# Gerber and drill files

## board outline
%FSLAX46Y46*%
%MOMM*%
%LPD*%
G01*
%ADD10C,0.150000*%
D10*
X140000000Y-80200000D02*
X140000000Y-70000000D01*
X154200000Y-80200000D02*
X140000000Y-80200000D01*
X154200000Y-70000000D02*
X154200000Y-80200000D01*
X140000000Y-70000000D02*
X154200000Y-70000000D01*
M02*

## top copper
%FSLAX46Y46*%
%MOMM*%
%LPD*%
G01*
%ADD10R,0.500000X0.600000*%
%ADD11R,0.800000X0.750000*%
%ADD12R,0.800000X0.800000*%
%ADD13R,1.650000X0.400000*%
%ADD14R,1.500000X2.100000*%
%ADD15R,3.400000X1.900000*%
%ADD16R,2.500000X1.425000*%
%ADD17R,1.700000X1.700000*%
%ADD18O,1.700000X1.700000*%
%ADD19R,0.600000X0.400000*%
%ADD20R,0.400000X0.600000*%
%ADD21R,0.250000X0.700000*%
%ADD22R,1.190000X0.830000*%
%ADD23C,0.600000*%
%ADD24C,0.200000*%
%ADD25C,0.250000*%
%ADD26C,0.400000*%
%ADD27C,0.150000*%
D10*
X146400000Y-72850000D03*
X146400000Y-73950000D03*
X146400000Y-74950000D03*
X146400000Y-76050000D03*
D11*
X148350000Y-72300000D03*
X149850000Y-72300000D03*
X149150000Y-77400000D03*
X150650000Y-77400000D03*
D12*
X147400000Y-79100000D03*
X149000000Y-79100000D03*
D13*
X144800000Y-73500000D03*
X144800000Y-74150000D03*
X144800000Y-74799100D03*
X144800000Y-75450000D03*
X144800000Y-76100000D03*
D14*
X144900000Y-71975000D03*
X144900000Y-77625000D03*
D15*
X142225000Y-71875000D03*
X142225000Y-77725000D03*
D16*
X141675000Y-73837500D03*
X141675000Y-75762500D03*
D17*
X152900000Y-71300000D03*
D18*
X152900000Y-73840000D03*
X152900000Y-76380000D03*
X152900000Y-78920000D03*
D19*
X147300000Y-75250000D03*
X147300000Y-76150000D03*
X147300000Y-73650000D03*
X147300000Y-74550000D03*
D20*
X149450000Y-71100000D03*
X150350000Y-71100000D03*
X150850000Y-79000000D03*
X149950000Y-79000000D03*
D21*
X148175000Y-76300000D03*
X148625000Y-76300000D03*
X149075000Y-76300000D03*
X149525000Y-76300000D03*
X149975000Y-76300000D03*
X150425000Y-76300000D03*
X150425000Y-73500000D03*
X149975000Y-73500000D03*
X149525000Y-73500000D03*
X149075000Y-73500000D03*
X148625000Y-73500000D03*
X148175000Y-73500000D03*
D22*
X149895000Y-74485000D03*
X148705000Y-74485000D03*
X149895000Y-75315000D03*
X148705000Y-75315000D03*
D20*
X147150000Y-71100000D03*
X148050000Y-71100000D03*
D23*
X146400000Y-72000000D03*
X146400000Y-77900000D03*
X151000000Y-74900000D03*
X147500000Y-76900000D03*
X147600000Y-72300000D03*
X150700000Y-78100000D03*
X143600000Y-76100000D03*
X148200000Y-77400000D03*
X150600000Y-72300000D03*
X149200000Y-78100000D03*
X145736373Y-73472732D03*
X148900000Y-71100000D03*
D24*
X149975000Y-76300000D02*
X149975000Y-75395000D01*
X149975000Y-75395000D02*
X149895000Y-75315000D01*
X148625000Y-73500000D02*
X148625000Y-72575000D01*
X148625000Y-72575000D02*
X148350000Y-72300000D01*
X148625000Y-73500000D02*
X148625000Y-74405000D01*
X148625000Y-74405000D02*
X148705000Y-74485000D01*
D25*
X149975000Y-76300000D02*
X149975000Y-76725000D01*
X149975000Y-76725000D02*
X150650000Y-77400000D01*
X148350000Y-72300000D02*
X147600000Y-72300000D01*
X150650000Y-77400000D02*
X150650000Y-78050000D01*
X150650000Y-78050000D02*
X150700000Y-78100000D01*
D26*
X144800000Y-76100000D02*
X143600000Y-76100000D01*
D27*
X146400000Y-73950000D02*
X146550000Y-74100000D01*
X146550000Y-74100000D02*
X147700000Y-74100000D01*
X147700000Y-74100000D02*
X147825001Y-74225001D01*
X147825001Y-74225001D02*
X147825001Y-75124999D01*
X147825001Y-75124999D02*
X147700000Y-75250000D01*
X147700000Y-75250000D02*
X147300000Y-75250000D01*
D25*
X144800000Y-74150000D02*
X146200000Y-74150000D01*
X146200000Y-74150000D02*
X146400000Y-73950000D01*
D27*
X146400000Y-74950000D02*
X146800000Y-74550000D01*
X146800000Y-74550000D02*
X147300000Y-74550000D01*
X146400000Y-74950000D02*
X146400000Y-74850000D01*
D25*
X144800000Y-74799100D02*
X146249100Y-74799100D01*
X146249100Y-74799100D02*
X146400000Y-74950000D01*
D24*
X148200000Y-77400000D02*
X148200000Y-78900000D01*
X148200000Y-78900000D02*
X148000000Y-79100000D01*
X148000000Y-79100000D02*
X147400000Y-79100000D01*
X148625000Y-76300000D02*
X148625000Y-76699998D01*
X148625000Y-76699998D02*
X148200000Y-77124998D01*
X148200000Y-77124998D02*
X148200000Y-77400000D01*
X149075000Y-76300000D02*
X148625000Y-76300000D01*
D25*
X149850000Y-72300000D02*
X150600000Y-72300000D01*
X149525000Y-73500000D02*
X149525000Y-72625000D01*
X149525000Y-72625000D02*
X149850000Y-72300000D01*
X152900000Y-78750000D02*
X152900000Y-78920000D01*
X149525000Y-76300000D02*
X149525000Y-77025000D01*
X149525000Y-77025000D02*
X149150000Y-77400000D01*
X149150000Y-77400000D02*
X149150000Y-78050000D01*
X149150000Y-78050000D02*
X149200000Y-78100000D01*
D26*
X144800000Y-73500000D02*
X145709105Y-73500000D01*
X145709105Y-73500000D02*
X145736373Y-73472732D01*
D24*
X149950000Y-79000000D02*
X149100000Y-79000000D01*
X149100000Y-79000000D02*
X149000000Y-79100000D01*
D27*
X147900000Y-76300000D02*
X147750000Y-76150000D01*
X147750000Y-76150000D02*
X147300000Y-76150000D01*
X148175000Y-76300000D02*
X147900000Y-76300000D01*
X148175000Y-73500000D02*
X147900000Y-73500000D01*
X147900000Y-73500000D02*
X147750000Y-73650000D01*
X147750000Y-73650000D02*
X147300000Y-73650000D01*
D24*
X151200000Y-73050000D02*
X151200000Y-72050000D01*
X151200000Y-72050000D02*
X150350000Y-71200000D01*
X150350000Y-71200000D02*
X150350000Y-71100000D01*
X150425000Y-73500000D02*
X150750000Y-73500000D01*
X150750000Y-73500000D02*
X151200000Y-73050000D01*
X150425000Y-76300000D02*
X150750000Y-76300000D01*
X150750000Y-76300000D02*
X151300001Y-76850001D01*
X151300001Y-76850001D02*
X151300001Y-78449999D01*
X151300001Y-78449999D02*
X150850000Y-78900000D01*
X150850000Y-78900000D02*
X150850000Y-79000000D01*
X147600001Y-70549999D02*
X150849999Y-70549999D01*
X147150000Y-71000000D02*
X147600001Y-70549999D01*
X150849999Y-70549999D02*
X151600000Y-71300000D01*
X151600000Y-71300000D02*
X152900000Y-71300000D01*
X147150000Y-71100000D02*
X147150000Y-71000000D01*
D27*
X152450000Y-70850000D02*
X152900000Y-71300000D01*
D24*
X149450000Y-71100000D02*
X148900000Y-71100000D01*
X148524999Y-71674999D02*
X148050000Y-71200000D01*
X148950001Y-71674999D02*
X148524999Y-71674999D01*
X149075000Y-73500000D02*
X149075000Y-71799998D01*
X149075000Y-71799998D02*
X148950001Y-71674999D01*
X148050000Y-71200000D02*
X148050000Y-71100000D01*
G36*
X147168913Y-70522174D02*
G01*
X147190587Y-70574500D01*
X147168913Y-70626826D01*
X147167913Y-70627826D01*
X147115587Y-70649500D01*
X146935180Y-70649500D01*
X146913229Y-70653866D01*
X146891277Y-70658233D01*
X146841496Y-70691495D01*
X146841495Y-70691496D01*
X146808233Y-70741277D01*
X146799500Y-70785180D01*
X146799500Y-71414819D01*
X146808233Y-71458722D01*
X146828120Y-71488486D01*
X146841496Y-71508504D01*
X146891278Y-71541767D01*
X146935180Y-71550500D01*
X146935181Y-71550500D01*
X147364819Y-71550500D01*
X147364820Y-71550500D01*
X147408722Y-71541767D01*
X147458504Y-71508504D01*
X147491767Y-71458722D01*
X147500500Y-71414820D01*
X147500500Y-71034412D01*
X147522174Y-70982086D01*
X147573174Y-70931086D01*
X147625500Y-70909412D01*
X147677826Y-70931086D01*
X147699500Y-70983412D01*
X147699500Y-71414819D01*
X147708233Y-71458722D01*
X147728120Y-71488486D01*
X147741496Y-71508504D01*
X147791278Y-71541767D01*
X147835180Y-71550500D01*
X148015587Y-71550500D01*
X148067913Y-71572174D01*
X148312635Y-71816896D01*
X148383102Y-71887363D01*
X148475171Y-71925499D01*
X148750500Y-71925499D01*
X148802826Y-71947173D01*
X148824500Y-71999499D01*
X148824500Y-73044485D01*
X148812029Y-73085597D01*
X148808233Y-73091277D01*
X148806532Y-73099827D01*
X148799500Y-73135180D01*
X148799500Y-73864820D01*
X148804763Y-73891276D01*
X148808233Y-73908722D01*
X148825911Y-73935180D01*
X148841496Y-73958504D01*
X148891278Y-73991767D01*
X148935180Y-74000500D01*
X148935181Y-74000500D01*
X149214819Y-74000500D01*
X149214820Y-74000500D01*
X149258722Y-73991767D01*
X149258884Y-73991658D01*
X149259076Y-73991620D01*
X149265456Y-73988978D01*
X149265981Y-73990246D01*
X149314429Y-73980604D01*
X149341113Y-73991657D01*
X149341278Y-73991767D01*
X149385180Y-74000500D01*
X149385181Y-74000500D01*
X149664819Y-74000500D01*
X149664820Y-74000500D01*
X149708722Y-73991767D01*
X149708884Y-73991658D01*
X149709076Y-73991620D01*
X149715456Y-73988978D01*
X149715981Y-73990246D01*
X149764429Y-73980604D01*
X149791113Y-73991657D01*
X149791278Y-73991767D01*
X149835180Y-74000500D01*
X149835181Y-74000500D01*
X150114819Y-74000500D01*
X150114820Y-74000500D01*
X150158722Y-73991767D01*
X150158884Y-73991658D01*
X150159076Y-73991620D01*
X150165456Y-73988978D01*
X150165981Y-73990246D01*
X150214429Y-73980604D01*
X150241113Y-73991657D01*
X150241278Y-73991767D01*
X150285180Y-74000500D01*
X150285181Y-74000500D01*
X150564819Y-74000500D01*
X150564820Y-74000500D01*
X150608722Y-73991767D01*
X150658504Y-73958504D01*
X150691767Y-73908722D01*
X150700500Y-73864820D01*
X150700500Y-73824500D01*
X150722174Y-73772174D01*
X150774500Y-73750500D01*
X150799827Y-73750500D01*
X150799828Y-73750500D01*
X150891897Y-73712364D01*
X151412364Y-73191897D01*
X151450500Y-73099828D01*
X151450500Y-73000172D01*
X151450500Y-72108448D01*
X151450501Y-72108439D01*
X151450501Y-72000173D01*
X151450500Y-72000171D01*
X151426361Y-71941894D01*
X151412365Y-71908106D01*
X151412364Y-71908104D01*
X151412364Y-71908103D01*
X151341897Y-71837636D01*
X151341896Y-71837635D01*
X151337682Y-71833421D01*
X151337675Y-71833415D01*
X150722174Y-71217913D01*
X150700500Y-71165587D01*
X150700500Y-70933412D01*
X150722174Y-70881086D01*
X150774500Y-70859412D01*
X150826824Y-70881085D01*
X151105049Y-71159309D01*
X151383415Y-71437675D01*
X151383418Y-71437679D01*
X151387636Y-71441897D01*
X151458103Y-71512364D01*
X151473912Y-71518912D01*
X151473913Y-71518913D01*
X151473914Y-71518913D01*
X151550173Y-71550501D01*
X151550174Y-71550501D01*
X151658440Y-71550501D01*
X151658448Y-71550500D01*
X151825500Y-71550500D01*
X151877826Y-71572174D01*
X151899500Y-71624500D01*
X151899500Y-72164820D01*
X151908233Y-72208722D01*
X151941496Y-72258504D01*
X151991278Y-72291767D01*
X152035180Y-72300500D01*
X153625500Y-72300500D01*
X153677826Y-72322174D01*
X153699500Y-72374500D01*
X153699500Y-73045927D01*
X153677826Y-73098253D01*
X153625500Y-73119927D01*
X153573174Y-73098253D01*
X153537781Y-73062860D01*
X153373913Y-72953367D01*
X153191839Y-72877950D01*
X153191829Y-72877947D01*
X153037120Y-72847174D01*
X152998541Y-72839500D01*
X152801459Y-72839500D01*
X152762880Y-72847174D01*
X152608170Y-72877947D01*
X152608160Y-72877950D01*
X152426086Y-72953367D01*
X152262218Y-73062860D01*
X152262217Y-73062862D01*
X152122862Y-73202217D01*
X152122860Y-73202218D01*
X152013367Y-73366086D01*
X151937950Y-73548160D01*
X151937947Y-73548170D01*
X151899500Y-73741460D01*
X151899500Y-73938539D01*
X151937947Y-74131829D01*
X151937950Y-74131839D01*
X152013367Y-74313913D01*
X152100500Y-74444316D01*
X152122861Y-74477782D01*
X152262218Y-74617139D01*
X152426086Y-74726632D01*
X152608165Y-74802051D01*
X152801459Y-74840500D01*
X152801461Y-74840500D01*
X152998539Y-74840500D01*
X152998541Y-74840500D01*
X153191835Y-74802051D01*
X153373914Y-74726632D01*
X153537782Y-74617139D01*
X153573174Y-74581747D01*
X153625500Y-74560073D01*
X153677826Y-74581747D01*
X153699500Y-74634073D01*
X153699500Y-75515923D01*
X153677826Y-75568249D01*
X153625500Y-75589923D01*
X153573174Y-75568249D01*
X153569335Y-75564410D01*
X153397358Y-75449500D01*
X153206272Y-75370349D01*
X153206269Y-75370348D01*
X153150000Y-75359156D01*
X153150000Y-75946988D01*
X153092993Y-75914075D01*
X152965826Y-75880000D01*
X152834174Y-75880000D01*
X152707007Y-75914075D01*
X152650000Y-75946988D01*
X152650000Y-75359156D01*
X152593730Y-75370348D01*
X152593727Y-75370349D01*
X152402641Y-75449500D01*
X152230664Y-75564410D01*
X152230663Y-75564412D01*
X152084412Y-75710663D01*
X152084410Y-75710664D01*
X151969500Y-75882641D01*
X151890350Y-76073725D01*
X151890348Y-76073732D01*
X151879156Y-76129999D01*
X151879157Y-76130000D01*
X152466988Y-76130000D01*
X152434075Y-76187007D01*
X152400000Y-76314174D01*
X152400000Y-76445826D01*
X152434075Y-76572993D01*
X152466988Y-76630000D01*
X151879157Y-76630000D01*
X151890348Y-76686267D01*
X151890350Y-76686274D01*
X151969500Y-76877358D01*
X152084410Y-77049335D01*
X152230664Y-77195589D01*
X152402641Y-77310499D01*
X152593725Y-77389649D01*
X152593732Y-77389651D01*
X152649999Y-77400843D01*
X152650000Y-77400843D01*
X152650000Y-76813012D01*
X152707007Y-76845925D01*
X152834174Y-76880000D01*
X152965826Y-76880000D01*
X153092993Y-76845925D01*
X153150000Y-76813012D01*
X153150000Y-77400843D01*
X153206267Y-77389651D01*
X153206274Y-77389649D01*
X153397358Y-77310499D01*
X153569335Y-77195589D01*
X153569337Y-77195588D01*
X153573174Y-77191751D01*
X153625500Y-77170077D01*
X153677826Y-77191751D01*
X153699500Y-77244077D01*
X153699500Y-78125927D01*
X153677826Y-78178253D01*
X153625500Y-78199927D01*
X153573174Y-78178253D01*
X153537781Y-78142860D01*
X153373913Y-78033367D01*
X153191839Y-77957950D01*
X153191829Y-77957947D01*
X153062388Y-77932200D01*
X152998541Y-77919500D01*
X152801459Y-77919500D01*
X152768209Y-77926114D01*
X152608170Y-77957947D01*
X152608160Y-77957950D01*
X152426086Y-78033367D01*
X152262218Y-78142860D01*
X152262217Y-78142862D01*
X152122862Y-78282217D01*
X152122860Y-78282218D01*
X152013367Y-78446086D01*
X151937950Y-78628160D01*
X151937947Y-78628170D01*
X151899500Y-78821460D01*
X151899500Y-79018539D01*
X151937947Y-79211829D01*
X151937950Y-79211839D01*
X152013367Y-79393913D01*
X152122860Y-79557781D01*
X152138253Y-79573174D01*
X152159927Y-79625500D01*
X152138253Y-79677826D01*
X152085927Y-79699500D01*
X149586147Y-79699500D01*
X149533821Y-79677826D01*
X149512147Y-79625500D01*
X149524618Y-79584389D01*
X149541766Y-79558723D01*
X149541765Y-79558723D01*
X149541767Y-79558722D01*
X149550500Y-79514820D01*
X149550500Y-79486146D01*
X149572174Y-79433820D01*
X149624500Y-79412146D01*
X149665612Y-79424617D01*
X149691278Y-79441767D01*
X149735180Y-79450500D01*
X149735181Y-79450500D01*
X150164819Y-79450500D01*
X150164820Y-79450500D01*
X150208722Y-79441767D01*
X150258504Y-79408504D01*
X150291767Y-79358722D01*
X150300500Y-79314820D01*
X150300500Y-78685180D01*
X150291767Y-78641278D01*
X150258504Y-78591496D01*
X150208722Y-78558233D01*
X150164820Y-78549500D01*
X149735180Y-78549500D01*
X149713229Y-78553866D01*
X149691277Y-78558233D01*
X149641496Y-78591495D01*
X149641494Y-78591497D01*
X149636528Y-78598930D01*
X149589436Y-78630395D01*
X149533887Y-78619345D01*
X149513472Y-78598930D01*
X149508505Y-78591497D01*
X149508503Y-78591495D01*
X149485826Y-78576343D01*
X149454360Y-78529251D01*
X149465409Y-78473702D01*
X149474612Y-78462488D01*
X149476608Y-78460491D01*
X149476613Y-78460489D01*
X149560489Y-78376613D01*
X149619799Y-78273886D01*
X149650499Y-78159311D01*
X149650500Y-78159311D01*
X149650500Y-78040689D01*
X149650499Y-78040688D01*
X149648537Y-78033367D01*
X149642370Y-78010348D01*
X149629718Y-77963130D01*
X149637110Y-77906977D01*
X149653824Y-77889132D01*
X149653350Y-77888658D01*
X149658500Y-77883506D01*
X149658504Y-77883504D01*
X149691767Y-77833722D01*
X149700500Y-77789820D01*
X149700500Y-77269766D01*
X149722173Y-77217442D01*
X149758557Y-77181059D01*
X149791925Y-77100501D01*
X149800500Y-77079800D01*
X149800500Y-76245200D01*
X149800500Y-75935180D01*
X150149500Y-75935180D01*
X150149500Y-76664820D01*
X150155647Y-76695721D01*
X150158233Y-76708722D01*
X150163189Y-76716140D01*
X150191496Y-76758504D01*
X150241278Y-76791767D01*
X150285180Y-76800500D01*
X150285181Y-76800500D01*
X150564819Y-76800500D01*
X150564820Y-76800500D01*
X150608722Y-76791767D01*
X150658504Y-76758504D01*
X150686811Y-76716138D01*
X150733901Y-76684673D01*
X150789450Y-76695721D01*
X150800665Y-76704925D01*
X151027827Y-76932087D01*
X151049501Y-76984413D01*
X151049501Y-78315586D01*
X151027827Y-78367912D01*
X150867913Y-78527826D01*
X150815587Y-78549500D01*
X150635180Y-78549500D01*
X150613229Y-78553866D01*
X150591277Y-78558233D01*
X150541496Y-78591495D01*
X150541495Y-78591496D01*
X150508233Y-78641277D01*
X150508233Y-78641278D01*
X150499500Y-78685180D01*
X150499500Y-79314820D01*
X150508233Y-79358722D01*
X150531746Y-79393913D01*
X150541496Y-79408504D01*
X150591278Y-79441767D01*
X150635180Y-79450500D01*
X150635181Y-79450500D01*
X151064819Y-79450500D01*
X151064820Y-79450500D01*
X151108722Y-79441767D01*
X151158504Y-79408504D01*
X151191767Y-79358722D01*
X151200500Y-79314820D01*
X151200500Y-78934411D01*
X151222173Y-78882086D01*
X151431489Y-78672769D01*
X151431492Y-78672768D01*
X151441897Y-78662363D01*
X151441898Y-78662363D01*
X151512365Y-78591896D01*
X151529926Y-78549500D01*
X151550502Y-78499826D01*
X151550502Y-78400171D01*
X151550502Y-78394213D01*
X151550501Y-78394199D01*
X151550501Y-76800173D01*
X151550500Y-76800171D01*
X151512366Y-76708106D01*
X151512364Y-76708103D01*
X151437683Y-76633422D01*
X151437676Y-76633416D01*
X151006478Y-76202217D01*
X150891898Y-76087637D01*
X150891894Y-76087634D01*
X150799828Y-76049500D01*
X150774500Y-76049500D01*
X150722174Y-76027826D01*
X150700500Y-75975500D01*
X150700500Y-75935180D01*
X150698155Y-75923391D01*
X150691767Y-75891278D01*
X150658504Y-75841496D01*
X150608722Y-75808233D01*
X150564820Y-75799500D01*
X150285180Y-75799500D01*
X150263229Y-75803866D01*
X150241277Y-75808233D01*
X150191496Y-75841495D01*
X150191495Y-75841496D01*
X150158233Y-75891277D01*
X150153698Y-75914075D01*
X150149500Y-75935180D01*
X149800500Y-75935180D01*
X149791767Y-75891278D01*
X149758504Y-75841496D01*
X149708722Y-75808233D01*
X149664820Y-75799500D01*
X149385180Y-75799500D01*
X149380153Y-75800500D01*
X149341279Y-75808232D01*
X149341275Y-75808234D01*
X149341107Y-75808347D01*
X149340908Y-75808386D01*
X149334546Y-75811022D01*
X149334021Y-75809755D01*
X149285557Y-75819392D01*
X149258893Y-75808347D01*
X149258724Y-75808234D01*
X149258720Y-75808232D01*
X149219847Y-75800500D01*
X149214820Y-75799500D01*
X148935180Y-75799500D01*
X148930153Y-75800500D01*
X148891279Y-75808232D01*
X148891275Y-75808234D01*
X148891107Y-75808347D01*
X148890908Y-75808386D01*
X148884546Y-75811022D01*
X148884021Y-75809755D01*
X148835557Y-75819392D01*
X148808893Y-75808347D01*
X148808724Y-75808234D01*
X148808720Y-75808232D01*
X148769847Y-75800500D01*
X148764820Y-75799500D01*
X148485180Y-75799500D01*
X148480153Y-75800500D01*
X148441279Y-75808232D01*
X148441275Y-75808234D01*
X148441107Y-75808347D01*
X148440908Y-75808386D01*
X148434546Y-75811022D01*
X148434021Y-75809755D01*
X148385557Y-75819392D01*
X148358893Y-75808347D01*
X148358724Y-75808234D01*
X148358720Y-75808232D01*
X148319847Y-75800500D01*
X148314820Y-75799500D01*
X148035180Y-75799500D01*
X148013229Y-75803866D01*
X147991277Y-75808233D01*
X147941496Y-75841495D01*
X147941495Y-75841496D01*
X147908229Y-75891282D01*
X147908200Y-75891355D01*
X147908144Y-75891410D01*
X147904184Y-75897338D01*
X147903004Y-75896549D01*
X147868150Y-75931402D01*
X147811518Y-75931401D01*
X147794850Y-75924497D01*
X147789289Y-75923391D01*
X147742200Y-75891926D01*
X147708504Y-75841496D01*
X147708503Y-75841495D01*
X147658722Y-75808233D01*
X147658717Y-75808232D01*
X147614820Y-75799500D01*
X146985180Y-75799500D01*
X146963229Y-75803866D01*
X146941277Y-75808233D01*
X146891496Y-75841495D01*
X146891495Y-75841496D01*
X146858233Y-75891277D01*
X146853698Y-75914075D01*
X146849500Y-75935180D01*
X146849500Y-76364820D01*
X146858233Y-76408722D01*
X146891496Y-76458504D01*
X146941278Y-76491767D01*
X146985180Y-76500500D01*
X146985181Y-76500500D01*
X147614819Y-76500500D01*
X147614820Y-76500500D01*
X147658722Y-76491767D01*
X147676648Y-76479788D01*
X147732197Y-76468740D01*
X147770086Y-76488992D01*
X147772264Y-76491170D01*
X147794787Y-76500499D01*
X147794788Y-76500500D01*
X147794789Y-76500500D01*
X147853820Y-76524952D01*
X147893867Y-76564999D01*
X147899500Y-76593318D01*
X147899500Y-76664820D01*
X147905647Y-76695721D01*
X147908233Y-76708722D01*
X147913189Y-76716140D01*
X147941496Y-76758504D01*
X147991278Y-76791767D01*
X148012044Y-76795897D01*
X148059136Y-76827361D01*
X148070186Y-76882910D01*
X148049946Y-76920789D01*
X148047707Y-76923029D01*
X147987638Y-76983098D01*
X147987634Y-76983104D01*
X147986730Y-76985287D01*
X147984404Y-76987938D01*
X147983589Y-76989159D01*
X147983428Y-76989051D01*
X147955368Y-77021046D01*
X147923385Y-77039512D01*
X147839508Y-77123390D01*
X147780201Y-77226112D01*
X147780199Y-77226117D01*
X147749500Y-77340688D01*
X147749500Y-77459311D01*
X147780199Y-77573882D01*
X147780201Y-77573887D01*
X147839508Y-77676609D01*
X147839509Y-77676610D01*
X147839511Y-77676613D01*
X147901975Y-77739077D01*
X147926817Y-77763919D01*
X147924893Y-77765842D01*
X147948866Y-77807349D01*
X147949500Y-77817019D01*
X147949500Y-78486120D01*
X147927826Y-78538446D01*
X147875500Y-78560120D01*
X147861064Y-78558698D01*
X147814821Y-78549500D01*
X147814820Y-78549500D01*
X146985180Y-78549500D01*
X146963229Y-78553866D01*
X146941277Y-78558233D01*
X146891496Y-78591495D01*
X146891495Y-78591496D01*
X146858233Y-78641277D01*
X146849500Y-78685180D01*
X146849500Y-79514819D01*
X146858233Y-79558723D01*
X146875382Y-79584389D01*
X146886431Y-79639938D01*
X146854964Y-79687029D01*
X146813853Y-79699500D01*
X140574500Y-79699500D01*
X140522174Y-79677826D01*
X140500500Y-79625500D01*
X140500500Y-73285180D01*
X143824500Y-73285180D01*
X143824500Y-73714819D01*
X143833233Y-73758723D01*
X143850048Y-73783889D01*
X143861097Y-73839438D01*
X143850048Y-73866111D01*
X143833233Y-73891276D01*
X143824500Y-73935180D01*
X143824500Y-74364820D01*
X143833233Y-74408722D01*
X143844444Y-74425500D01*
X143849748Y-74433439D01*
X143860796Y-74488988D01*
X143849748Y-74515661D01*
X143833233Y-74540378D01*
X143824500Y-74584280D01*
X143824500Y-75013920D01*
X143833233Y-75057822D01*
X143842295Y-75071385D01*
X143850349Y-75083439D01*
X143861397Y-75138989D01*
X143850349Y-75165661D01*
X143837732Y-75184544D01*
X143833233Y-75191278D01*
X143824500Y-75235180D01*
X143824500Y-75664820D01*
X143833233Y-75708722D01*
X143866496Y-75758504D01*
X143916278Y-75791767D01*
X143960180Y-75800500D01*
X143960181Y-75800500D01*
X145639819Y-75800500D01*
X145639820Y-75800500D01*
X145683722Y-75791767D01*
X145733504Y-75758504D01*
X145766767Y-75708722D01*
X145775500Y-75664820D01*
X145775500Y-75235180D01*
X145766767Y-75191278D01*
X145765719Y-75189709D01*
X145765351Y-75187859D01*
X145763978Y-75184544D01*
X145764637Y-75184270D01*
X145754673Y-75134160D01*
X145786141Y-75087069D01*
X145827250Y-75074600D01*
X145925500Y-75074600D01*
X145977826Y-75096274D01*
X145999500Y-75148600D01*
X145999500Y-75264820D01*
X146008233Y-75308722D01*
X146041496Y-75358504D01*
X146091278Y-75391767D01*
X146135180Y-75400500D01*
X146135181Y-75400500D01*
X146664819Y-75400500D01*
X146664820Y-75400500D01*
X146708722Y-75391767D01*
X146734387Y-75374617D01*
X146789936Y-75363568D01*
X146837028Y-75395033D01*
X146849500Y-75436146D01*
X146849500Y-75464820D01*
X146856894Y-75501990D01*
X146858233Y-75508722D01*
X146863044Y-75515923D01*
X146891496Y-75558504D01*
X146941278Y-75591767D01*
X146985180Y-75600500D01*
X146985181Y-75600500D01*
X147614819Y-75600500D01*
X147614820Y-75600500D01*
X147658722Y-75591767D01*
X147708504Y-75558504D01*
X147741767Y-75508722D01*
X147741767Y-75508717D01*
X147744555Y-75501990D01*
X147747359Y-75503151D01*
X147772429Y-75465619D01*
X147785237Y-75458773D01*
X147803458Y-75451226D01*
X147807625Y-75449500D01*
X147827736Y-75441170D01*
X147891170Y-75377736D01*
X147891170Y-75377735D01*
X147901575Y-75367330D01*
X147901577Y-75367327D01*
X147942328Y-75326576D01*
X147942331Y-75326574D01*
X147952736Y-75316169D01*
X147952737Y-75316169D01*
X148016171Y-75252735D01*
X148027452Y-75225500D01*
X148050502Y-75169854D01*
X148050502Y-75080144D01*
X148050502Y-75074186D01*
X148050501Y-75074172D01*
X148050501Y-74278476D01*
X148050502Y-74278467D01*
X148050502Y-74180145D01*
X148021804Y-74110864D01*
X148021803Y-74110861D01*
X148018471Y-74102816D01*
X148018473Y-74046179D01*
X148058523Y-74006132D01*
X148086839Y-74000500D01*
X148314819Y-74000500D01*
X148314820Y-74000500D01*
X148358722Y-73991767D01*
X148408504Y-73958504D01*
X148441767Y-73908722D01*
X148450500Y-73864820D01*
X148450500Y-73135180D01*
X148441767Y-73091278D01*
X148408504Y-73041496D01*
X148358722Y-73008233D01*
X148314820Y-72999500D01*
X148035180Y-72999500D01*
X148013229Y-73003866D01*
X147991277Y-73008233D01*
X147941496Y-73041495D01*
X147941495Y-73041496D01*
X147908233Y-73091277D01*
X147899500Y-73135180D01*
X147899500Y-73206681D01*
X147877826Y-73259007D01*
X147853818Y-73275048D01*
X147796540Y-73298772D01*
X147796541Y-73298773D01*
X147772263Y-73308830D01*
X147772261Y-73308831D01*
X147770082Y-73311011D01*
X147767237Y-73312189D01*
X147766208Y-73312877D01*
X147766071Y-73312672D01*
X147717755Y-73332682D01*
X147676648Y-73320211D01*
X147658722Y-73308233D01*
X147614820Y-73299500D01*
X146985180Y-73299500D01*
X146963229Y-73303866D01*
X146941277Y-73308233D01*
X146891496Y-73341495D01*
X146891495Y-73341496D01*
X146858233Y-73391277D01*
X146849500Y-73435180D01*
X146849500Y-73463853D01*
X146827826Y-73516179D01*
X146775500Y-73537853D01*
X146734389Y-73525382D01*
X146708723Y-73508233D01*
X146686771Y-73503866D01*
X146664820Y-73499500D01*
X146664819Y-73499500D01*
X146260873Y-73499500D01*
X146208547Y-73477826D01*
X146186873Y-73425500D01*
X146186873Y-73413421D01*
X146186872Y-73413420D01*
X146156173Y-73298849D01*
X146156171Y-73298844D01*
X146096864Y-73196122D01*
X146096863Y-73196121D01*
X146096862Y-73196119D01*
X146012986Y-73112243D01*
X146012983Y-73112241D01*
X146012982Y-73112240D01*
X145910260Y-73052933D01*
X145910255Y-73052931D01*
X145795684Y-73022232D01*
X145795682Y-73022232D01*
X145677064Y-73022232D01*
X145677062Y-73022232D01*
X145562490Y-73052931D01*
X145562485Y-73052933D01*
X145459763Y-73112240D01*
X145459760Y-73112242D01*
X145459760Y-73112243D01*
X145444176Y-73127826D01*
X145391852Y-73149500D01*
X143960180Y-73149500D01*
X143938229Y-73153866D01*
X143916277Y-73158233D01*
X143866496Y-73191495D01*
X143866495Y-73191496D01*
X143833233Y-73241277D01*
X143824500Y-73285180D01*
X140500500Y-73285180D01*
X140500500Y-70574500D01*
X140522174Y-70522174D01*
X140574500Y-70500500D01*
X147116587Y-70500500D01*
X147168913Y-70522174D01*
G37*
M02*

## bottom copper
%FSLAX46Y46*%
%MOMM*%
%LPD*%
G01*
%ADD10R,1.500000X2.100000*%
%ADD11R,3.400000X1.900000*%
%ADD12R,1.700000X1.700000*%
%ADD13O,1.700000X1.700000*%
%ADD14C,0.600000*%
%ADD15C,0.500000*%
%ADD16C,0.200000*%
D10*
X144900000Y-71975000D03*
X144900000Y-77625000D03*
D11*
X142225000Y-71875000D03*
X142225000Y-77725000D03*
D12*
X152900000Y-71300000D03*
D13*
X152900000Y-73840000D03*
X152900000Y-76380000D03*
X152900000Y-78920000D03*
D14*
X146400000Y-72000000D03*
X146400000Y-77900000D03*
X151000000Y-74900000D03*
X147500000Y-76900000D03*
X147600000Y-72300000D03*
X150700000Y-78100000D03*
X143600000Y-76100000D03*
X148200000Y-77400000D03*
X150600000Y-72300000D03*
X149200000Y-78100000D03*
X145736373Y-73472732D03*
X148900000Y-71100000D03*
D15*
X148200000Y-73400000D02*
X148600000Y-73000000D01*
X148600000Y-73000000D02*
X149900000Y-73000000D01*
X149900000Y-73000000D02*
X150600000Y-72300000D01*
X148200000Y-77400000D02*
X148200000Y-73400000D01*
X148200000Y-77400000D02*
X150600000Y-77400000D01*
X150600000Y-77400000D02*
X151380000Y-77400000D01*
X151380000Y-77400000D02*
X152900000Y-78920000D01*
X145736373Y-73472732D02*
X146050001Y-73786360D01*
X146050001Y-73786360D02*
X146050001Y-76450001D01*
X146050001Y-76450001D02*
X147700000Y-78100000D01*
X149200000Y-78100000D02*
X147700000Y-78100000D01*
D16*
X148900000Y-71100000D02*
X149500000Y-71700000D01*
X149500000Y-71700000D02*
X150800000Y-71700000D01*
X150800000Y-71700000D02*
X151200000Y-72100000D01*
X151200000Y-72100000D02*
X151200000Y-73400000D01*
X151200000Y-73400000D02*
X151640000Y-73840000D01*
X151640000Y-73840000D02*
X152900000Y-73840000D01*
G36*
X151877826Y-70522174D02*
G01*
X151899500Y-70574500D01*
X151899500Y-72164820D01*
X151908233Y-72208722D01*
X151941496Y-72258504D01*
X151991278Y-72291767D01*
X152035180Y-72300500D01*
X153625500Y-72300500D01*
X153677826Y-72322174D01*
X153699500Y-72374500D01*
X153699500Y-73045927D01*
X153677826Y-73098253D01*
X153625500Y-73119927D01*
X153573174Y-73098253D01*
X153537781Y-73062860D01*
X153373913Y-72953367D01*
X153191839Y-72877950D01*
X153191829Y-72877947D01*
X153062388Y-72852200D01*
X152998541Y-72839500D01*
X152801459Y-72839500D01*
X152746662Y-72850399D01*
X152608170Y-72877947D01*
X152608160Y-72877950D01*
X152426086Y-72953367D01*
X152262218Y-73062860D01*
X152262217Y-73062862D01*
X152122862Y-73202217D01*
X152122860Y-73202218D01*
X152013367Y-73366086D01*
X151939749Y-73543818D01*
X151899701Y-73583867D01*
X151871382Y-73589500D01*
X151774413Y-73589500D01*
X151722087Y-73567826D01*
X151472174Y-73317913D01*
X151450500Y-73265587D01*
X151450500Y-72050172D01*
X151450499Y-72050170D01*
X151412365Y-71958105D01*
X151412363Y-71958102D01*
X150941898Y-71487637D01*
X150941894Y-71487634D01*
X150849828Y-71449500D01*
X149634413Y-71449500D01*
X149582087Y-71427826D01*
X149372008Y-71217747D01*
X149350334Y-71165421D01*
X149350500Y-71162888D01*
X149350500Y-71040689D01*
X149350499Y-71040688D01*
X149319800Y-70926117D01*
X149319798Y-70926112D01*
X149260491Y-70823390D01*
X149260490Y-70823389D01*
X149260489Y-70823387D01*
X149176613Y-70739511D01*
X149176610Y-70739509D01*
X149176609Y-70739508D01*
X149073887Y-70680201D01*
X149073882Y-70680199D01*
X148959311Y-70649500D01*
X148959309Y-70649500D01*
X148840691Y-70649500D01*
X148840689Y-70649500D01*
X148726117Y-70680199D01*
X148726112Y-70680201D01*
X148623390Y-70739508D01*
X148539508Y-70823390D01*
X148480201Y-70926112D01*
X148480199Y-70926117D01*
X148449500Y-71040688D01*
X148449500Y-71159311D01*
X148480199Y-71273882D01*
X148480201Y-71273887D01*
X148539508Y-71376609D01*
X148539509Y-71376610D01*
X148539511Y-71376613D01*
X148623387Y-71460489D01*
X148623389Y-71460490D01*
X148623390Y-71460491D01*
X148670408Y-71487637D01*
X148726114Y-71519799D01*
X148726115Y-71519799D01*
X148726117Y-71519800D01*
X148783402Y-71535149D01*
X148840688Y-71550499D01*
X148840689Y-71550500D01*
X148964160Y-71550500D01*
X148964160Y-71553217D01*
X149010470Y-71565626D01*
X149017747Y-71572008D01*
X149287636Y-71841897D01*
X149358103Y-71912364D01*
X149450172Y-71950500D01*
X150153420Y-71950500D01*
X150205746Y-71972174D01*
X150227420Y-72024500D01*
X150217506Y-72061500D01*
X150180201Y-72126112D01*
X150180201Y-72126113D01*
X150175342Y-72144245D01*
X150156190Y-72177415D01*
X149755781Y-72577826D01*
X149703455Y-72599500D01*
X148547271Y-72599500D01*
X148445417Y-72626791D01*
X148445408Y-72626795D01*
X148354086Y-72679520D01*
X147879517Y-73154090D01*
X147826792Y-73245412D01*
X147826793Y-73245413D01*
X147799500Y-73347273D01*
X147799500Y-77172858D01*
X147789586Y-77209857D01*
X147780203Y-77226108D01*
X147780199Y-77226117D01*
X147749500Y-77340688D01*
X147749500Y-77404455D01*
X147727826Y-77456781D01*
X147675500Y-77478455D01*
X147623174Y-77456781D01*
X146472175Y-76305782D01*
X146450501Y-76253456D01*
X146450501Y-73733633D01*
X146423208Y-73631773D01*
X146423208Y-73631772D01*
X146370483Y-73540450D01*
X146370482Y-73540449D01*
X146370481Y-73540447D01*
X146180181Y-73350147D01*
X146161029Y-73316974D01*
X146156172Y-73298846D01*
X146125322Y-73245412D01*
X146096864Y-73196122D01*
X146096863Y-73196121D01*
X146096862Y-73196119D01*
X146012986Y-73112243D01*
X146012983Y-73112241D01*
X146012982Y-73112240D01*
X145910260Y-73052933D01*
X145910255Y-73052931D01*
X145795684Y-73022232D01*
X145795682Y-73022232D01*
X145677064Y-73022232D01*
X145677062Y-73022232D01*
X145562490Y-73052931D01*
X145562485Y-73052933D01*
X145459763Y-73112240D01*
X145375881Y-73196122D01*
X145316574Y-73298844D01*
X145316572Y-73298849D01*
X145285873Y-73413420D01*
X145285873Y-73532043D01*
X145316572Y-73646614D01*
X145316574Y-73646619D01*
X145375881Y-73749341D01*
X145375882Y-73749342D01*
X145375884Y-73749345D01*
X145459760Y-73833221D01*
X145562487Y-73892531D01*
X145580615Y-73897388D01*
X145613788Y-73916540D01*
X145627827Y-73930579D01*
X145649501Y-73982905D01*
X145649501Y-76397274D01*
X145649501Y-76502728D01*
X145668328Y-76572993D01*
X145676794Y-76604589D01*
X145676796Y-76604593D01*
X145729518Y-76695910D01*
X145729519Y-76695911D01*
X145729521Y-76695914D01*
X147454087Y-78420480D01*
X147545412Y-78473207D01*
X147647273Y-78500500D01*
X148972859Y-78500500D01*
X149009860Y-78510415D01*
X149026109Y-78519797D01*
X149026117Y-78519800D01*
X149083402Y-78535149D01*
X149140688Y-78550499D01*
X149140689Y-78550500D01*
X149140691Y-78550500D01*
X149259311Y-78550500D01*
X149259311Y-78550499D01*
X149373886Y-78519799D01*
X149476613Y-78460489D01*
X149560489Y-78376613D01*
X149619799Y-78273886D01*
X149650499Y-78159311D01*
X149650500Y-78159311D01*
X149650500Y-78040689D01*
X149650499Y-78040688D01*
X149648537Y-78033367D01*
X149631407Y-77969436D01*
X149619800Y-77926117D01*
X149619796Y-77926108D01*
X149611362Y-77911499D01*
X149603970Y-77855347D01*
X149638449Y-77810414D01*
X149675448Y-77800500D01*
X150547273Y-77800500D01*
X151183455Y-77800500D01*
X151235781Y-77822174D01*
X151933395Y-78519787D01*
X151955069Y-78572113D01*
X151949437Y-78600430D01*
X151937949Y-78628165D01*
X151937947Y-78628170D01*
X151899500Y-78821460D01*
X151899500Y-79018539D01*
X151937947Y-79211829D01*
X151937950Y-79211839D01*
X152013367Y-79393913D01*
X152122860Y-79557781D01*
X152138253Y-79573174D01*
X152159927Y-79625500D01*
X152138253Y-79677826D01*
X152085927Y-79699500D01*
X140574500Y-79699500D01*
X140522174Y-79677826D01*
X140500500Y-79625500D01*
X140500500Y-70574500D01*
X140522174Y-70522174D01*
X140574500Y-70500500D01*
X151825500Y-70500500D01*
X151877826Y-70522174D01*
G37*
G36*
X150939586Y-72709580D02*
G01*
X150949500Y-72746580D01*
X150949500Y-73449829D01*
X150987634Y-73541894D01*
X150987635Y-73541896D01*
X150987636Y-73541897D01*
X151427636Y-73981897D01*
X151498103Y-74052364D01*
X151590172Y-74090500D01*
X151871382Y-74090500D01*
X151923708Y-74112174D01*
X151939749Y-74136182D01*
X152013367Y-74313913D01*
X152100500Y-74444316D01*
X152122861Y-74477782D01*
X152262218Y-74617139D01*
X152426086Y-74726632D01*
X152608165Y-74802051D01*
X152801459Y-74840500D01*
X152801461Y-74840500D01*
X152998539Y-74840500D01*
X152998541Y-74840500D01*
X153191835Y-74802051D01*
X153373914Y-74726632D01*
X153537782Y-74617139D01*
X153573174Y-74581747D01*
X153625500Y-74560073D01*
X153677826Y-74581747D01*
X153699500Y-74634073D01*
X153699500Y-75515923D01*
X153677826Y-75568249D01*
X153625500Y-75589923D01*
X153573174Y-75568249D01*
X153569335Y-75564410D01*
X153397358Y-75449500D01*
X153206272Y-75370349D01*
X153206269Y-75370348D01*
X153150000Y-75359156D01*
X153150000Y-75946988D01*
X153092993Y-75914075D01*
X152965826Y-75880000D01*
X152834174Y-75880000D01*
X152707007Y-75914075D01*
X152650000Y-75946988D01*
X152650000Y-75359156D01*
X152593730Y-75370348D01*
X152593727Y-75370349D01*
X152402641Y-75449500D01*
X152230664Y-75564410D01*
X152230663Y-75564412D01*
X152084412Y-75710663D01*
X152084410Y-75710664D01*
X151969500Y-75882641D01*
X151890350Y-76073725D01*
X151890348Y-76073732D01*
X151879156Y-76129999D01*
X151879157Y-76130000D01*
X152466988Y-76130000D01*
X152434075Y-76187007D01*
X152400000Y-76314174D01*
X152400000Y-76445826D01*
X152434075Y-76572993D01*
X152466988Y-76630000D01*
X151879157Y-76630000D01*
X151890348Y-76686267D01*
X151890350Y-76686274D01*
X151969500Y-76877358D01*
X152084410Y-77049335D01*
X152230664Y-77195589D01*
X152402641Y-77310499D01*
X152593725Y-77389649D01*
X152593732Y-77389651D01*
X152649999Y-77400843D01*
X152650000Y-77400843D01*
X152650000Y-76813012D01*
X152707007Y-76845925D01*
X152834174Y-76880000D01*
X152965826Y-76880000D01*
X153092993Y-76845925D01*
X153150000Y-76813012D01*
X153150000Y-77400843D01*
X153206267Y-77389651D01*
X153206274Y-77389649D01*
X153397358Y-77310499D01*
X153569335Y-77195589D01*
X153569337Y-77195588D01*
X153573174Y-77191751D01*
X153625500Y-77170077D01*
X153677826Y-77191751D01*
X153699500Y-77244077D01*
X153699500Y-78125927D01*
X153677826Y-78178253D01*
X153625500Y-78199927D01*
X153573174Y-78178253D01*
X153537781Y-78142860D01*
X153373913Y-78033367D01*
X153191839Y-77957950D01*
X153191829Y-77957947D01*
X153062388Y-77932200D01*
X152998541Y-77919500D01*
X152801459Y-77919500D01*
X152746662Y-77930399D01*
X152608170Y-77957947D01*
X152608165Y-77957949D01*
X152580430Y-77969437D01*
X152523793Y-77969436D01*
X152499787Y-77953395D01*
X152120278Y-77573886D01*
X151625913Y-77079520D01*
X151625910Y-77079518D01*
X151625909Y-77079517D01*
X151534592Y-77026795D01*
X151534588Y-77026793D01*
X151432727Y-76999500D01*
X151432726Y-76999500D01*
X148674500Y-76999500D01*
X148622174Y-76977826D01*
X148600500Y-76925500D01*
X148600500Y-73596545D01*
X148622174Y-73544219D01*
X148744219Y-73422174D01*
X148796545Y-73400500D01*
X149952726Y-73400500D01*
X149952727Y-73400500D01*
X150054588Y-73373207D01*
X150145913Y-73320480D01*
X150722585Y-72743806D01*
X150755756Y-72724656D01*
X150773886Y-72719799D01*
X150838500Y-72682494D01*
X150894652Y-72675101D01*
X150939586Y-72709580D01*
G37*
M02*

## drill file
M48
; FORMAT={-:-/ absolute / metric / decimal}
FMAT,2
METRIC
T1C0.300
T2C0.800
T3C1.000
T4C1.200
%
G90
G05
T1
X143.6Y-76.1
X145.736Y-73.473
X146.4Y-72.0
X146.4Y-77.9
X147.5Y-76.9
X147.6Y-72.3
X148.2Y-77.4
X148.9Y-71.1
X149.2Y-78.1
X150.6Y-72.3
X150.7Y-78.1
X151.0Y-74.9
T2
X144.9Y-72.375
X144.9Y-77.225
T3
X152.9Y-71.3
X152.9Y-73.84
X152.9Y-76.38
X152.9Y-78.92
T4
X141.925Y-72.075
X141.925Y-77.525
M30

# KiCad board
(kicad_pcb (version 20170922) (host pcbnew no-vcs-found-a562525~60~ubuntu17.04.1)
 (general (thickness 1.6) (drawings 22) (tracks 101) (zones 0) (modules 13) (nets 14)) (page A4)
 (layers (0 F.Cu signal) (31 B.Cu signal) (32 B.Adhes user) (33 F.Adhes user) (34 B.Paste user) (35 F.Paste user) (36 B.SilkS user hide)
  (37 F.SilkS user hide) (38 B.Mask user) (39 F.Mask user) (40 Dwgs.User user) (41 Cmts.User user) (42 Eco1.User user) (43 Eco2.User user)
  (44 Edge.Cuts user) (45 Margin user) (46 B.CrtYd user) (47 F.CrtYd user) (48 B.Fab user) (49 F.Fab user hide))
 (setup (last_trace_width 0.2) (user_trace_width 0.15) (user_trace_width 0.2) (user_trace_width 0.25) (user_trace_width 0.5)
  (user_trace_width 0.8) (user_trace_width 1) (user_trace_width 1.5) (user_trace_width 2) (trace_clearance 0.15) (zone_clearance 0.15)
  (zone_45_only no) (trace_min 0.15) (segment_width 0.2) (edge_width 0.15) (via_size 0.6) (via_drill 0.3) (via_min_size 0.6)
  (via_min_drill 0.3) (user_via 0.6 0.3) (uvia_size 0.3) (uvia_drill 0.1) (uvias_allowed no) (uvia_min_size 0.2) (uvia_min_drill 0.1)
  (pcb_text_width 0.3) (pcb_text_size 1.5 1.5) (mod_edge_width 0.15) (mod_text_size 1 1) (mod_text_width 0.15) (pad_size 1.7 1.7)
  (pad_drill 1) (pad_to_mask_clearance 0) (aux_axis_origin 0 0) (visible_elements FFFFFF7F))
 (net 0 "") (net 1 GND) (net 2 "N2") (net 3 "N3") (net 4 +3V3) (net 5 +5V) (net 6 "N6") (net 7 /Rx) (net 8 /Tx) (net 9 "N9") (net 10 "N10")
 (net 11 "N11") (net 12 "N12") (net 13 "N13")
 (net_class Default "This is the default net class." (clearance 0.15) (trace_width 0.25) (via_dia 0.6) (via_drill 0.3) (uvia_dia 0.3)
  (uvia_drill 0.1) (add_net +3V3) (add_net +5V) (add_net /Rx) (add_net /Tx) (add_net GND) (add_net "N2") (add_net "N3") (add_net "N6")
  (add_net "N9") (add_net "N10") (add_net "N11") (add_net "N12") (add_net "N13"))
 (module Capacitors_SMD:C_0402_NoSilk (layer F.Cu) (at 146.4 73.4 90)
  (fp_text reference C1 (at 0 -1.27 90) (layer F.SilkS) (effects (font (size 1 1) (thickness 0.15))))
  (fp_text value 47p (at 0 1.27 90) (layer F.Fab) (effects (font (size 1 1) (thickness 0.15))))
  (pad 2 smd rect (at 0.55 0 90) (size 0.6 0.5) (layers F.Cu F.Paste F.Mask) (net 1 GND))
  (pad 1 smd rect (at -0.55 0 90) (size 0.6 0.5) (layers F.Cu F.Paste F.Mask) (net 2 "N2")))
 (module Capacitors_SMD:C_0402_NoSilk (layer F.Cu) (at 146.4 75.5 270)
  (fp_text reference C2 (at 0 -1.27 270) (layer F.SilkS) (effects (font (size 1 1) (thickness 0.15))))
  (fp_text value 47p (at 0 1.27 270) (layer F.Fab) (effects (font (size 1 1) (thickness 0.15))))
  (pad 1 smd rect (at -0.55 0 270) (size 0.6 0.5) (layers F.Cu F.Paste F.Mask) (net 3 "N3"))
  (pad 2 smd rect (at 0.55 0 270) (size 0.6 0.5) (layers F.Cu F.Paste F.Mask) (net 1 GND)))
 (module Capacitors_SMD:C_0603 (layer F.Cu) (at 149.1 72.3 180)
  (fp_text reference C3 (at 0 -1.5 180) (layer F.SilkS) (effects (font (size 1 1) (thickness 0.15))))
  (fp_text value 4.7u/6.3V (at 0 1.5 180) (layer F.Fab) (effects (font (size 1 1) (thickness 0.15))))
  (pad 2 smd rect (at 0.75 0 180) (size 0.8 0.75) (layers F.Cu F.Paste F.Mask) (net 1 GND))
  (pad 1 smd rect (at -0.75 0 180) (size 0.8 0.75) (layers F.Cu F.Paste F.Mask) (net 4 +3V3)))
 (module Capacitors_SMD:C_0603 (layer F.Cu) (at 149.9 77.4)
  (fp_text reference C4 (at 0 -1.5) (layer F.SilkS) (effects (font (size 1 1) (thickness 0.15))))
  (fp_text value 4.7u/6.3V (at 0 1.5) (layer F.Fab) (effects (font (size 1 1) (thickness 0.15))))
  (pad 1 smd rect (at -0.75 0) (size 0.8 0.75) (layers F.Cu F.Paste F.Mask) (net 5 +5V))
  (pad 2 smd rect (at 0.75 0) (size 0.8 0.75) (layers F.Cu F.Paste F.Mask) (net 1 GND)))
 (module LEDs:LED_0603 (layer F.Cu) (at 148.2 79.1 180)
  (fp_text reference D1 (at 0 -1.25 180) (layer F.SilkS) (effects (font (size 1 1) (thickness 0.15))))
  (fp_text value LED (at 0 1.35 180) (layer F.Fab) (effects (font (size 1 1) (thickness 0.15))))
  (pad 2 smd rect (at 0.8 0) (size 0.8 0.8) (layers F.Cu F.Paste F.Mask) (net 4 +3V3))
  (pad 1 smd rect (at -0.8 0) (size 0.8 0.8) (layers F.Cu F.Paste F.Mask) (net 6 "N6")))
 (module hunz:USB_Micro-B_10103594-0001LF (layer F.Cu) (at 142.8 74.8 180)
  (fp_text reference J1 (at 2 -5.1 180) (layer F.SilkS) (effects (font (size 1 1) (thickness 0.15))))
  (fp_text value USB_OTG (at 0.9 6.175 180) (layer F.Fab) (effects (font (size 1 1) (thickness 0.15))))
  (pad 1 smd rect (at -2 1.3) (size 1.65 0.4) (layers F.Cu F.Paste F.Mask) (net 5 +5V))
  (pad 2 smd rect (at -2 0.65) (size 1.65 0.4) (layers F.Cu F.Paste F.Mask) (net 2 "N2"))
  (pad 3 smd rect (at -2 0.0009) (size 1.65 0.4) (layers F.Cu F.Paste F.Mask) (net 3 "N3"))
  (pad 4 smd rect (at -2 -0.65) (size 1.65 0.4) (layers F.Cu F.Paste F.Mask))
  (pad 5 smd rect (at -2 -1.3) (size 1.65 0.4) (layers F.Cu F.Paste F.Mask) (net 1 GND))
  (pad 6 thru_hole rect (at -2.1 2.425) (size 1.5 2.1) (drill 0.8 (offset 0 -0.4)) (layers *.Cu *.Mask F.Paste) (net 1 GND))
  (pad 6 thru_hole rect (at -2.1 -2.425) (size 1.5 2.1) (drill 0.8 (offset 0 0.4)) (layers *.Cu *.Mask F.Paste) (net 1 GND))
  (pad 6 thru_hole rect (at 0.875 2.725) (size 3.4 1.9) (drill 1.2 (offset 0.3 -0.2)) (layers *.Cu *.Mask F.Paste) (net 1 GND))
  (pad 6 thru_hole rect (at 0.875 -2.725) (size 3.4 1.9) (drill 1.2 (offset 0.3 0.2)) (layers *.Cu *.Mask F.Paste) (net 1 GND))
  (pad 6 smd rect (at 1.125 0.9625) (size 2.5 1.425) (layers F.Cu F.Paste F.Mask) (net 1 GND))
  (pad 6 smd rect (at 1.125 -0.9625) (size 2.5 1.425) (layers F.Cu F.Paste F.Mask) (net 1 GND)))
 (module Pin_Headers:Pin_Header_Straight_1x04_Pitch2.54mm (layer F.Cu) (at 152.9 71.3)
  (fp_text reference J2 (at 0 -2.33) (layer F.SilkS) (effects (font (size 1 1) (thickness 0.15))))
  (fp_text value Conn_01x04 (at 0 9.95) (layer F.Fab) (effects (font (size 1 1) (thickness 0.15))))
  (pad 1 thru_hole rect (at 0 0) (size 1.7 1.7) (drill 1) (layers *.Cu *.Mask) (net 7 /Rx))
  (pad 2 thru_hole oval (at 0 2.54) (size 1.7 1.7) (drill 1) (layers *.Cu *.Mask) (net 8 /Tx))
  (pad 3 thru_hole oval (at 0 5.08) (size 1.7 1.7) (drill 1) (layers *.Cu *.Mask) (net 1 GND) (zone_connect 1) (thermal_width 0.5)
   (thermal_gap 0.2))
  (pad 4 thru_hole oval (at 0 7.62) (size 1.7 1.7) (drill 1) (layers *.Cu *.Mask) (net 4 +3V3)))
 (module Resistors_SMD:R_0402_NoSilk (layer F.Cu) (at 147.3 75.7 90)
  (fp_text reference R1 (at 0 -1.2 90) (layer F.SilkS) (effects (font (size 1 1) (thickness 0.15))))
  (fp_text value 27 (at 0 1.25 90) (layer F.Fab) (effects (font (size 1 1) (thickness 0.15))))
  (pad 2 smd rect (at 0.45 0 90) (size 0.4 0.6) (layers F.Cu F.Paste F.Mask) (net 2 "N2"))
  (pad 1 smd rect (at -0.45 0 90) (size 0.4 0.6) (layers F.Cu F.Paste F.Mask) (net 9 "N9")))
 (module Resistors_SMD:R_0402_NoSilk (layer F.Cu) (at 147.3 74.1 270)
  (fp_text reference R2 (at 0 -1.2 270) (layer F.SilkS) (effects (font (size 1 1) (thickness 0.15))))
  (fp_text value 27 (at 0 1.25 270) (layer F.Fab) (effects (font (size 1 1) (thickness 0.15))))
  (pad 1 smd rect (at -0.45 0 270) (size 0.4 0.6) (layers F.Cu F.Paste F.Mask) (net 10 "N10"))
  (pad 2 smd rect (at 0.45 0 270) (size 0.4 0.6) (layers F.Cu F.Paste F.Mask) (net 3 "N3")))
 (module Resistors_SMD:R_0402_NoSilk (layer F.Cu) (at 149.9 71.1)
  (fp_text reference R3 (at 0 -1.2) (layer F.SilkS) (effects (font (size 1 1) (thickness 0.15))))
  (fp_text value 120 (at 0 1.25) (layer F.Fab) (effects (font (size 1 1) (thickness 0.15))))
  (pad 1 smd rect (at -0.45 0) (size 0.4 0.6) (layers F.Cu F.Paste F.Mask) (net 8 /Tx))
  (pad 2 smd rect (at 0.45 0) (size 0.4 0.6) (layers F.Cu F.Paste F.Mask) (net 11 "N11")))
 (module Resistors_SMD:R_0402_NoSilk (layer F.Cu) (at 150.4 79)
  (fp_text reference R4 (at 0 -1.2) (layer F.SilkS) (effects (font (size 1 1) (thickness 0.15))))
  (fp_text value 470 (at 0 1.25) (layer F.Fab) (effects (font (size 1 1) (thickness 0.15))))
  (pad 2 smd rect (at 0.45 0) (size 0.4 0.6) (layers F.Cu F.Paste F.Mask) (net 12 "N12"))
  (pad 1 smd rect (at -0.45 0) (size 0.4 0.6) (layers F.Cu F.Paste F.Mask) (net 6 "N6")))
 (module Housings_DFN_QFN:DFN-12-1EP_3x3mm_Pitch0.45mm (layer F.Cu) (at 149.3 74.9 90)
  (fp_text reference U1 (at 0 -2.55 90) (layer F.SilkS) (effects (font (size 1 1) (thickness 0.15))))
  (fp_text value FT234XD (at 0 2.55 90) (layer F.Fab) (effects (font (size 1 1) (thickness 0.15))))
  (pad 1 smd rect (at -1.4 -1.125 90) (size 0.7 0.25) (layers F.Cu F.Paste F.Mask) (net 9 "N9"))
  (pad 2 smd rect (at -1.4 -0.675 90) (size 0.7 0.25) (layers F.Cu F.Paste F.Mask) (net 4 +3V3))
  (pad 3 smd rect (at -1.4 -0.225 90) (size 0.7 0.25) (layers F.Cu F.Paste F.Mask) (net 4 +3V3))
  (pad 4 smd rect (at -1.4 0.225 90) (size 0.7 0.25) (layers F.Cu F.Paste F.Mask) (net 5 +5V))
  (pad 5 smd rect (at -1.4 0.675 90) (size 0.7 0.25) (layers F.Cu F.Paste F.Mask) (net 1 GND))
  (pad 6 smd rect (at -1.4 1.125 90) (size 0.7 0.25) (layers F.Cu F.Paste F.Mask) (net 12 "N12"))
  (pad 7 smd rect (at 1.4 1.125 90) (size 0.7 0.25) (layers F.Cu F.Paste F.Mask) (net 11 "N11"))
  (pad 8 smd rect (at 1.4 0.675 90) (size 0.7 0.25) (layers F.Cu F.Paste F.Mask))
  (pad 9 smd rect (at 1.4 0.225 90) (size 0.7 0.25) (layers F.Cu F.Paste F.Mask) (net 4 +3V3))
  (pad 10 smd rect (at 1.4 -0.225 90) (size 0.7 0.25) (layers F.Cu F.Paste F.Mask) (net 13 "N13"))
  (pad 11 smd rect (at 1.4 -0.675 90) (size 0.7 0.25) (layers F.Cu F.Paste F.Mask) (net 1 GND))
  (pad 12 smd rect (at 1.4 -1.125 90) (size 0.7 0.25) (layers F.Cu F.Paste F.Mask) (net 10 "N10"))
  (pad 13 smd rect (at 0.415 0.595 90) (size 0.83 1.19) (layers F.Cu F.Paste F.Mask) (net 1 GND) (solder_paste_margin_ratio -0.2))
  (pad 13 smd rect (at 0.415 -0.595 90) (size 0.83 1.19) (layers F.Cu F.Paste F.Mask) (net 1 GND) (solder_paste_margin_ratio -0.2))
  (pad 13 smd rect (at -0.415 0.595 90) (size 0.83 1.19) (layers F.Cu F.Paste F.Mask) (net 1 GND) (solder_paste_margin_ratio -0.2))
  (pad 13 smd rect (at -0.415 -0.595 90) (size 0.83 1.19) (layers F.Cu F.Paste F.Mask) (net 1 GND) (solder_paste_margin_ratio -0.2)))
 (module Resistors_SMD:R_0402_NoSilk (layer F.Cu) (at 147.6 71.1)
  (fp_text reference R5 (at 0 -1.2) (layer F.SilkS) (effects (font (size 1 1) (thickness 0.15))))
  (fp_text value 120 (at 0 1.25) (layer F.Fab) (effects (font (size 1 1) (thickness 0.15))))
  (pad 1 smd rect (at -0.45 0) (size 0.4 0.6) (layers F.Cu F.Paste F.Mask) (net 7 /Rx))
  (pad 2 smd rect (at 0.45 0) (size 0.4 0.6) (layers F.Cu F.Paste F.Mask) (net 13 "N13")))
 (gr_line (start 140 80.2) (end 140 70) (layer Edge.Cuts) (width 0.15))
 (gr_line (start 154.2 80.2) (end 140 80.2) (layer Edge.Cuts) (width 0.15))
 (gr_line (start 154.2 70) (end 154.2 80.2) (layer Edge.Cuts) (width 0.15))
 (gr_line (start 140 70) (end 154.2 70) (layer Edge.Cuts) (width 0.15))
 (via (at 146.4 72) (size 0.6) (drill 0.3) (layers F.Cu B.Cu) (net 1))
 (via (at 146.4 77.9) (size 0.6) (drill 0.3) (layers F.Cu B.Cu) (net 1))
 (via (at 151 74.9) (size 0.6) (drill 0.3) (layers F.Cu B.Cu) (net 1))
 (via (at 147.5 76.9) (size 0.6) (drill 0.3) (layers F.Cu B.Cu) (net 1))
 (segment (start 149.975 76.3) (end 149.975 75.395) (width 0.2) (layer F.Cu) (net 1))
 (segment (start 149.975 75.395) (end 149.895 75.315) (width 0.2) (layer F.Cu) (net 1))
 (segment (start 148.625 73.5) (end 148.625 72.575) (width 0.2) (layer F.Cu) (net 1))
 (segment (start 148.625 72.575) (end 148.35 72.3) (width 0.2) (layer F.Cu) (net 1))
 (segment (start 148.625 73.5) (end 148.625 74.405) (width 0.2) (layer F.Cu) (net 1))
 (segment (start 148.625 74.405) (end 148.705 74.485) (width 0.2) (layer F.Cu) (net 1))
 (segment (start 149.975 76.3) (end 149.975 76.725) (width 0.25) (layer F.Cu) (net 1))
 (segment (start 149.975 76.725) (end 150.65 77.4) (width 0.25) (layer F.Cu) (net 1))
 (segment (start 148.35 72.3) (end 147.6 72.3) (width 0.25) (layer F.Cu) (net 1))
 (via (at 147.6 72.3) (size 0.6) (drill 0.3) (layers F.Cu B.Cu) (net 1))
 (segment (start 150.65 77.4) (end 150.65 78.05) (width 0.25) (layer F.Cu) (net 1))
 (segment (start 150.65 78.05) (end 150.7 78.1) (width 0.25) (layer F.Cu) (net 1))
 (via (at 150.7 78.1) (size 0.6) (drill 0.3) (layers F.Cu B.Cu) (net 1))
 (segment (start 144.8 76.1) (end 143.6 76.1) (width 0.4) (layer F.Cu) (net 1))
 (via (at 143.6 76.1) (size 0.6) (drill 0.3) (layers F.Cu B.Cu) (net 1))
 (segment (start 146.4 73.95) (end 146.55 74.1) (width 0.15) (layer F.Cu) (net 2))
 (segment (start 146.55 74.1) (end 147.7 74.1) (width 0.15) (layer F.Cu) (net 2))
 (segment (start 147.7 74.1) (end 147.825001 74.225001) (width 0.15) (layer F.Cu) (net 2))
 (segment (start 147.825001 74.225001) (end 147.825001 75.124999) (width 0.15) (layer F.Cu) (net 2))
 (segment (start 147.825001 75.124999) (end 147.7 75.25) (width 0.15) (layer F.Cu) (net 2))
 (segment (start 147.7 75.25) (end 147.3 75.25) (width 0.15) (layer F.Cu) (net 2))
 (segment (start 144.8 74.15) (end 146.2 74.15) (width 0.25) (layer F.Cu) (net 2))
 (segment (start 146.2 74.15) (end 146.4 73.95) (width 0.25) (layer F.Cu) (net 2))
 (segment (start 146.4 74.95) (end 146.8 74.55) (width 0.15) (layer F.Cu) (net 3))
 (segment (start 146.8 74.55) (end 147.3 74.55) (width 0.15) (layer F.Cu) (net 3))
 (segment (start 146.4 74.95) (end 146.4 74.85) (width 0.15) (layer F.Cu) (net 3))
 (segment (start 144.8 74.7991) (end 146.2491 74.7991) (width 0.25) (layer F.Cu) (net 3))
 (segment (start 146.2491 74.7991) (end 146.4 74.95) (width 0.25) (layer F.Cu) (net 3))
 (segment (start 148.2 73.4) (end 148.6 73) (width 0.5) (layer B.Cu) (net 4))
 (segment (start 148.6 73) (end 149.9 73) (width 0.5) (layer B.Cu) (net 4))
 (segment (start 149.9 73) (end 150.6 72.3) (width 0.5) (layer B.Cu) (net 4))
 (segment (start 148.2 77.4) (end 148.2 73.4) (width 0.5) (layer B.Cu) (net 4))
 (segment (start 148.2 77.4) (end 148.2 78.9) (width 0.2) (layer F.Cu) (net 4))
 (segment (start 148.2 78.9) (end 148 79.1) (width 0.2) (layer F.Cu) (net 4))
 (segment (start 148 79.1) (end 147.4 79.1) (width 0.2) (layer F.Cu) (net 4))
 (segment (start 148.2 77.4) (end 150.6 77.4) (width 0.5) (layer B.Cu) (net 4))
 (segment (start 150.6 77.4) (end 151.38 77.4) (width 0.5) (layer B.Cu) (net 4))
 (segment (start 151.38 77.4) (end 152.9 78.92) (width 0.5) (layer B.Cu) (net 4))
 (segment (start 148.625 76.3) (end 148.625 76.699998) (width 0.2) (layer F.Cu) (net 4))
 (segment (start 148.625 76.699998) (end 148.2 77.124998) (width 0.2) (layer F.Cu) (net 4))
 (segment (start 148.2 77.124998) (end 148.2 77.4) (width 0.2) (layer F.Cu) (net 4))
 (via (at 148.2 77.4) (size 0.6) (drill 0.3) (layers F.Cu B.Cu) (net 4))
 (segment (start 149.075 76.3) (end 148.625 76.3) (width 0.2) (layer F.Cu) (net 4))
 (segment (start 149.85 72.3) (end 150.6 72.3) (width 0.25) (layer F.Cu) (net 4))
 (via (at 150.6 72.3) (size 0.6) (drill 0.3) (layers F.Cu B.Cu) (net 4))
 (segment (start 149.525 73.5) (end 149.525 72.625) (width 0.25) (layer F.Cu) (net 4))
 (segment (start 149.525 72.625) (end 149.85 72.3) (width 0.25) (layer F.Cu) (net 4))
 (segment (start 152.9 78.75) (end 152.9 78.92) (width 0.25) (layer F.Cu) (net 4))
 (segment (start 145.736373 73.472732) (end 146.050001 73.78636) (width 0.5) (layer B.Cu) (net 5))
 (segment (start 146.050001 73.78636) (end 146.050001 76.450001) (width 0.5) (layer B.Cu) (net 5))
 (segment (start 146.050001 76.450001) (end 147.7 78.1) (width 0.5) (layer B.Cu) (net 5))
 (segment (start 149.2 78.1) (end 147.7 78.1) (width 0.5) (layer B.Cu) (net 5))
 (segment (start 149.525 76.3) (end 149.525 77.025) (width 0.25) (layer F.Cu) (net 5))
 (segment (start 149.525 77.025) (end 149.15 77.4) (width 0.25) (layer F.Cu) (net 5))
 (segment (start 149.15 77.4) (end 149.15 78.05) (width 0.25) (layer F.Cu) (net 5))
 (segment (start 149.15 78.05) (end 149.2 78.1) (width 0.25) (layer F.Cu) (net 5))
 (via (at 149.2 78.1) (size 0.6) (drill 0.3) (layers F.Cu B.Cu) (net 5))
 (segment (start 144.8 73.5) (end 145.709105 73.5) (width 0.4) (layer F.Cu) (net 5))
 (segment (start 145.709105 73.5) (end 145.736373 73.472732) (width 0.4) (layer F.Cu) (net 5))
 (via (at 145.736373 73.472732) (size 0.6) (drill 0.3) (layers F.Cu B.Cu) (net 5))
 (segment (start 149.95 79) (end 149.1 79) (width 0.2) (layer F.Cu) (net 6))
 (segment (start 149.1 79) (end 149 79.1) (width 0.2) (layer F.Cu) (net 6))
 (segment (start 147.9 76.3) (end 147.75 76.15) (width 0.15) (layer F.Cu) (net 9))
 (segment (start 147.75 76.15) (end 147.3 76.15) (width 0.15) (layer F.Cu) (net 9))
 (segment (start 148.175 76.3) (end 147.9 76.3) (width 0.15) (layer F.Cu) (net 9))
 (segment (start 148.175 73.5) (end 147.9 73.5) (width 0.15) (layer F.Cu) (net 10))
 (segment (start 147.9 73.5) (end 147.75 73.65) (width 0.15) (layer F.Cu) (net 10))
 (segment (start 147.75 73.65) (end 147.3 73.65) (width 0.15) (layer F.Cu) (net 10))
 (segment (start 151.2 73.05) (end 151.2 72.05) (width 0.2) (layer F.Cu) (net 11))
 (segment (start 151.2 72.05) (end 150.35 71.2) (width 0.2) (layer F.Cu) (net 11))
 (segment (start 150.35 71.2) (end 150.35 71.1) (width 0.2) (layer F.Cu) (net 11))
 (segment (start 150.425 73.5) (end 150.75 73.5) (width 0.2) (layer F.Cu) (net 11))
 (segment (start 150.75 73.5) (end 151.2 73.05) (width 0.2) (layer F.Cu) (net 11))
 (segment (start 150.425 76.3) (end 150.75 76.3) (width 0.2) (layer F.Cu) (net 12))
 (segment (start 150.75 76.3) (end 151.300001 76.850001) (width 0.2) (layer F.Cu) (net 12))
 (segment (start 151.300001 76.850001) (end 151.300001 78.449999) (width 0.2) (layer F.Cu) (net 12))
 (segment (start 151.300001 78.449999) (end 150.85 78.9) (width 0.2) (layer F.Cu) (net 12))
 (segment (start 150.85 78.9) (end 150.85 79) (width 0.2) (layer F.Cu) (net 12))
 (segment (start 147.600001 70.549999) (end 150.849999 70.549999) (width 0.2) (layer F.Cu) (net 7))
 (segment (start 147.15 71) (end 147.600001 70.549999) (width 0.2) (layer F.Cu) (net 7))
 (segment (start 150.849999 70.549999) (end 151.6 71.3) (width 0.2) (layer F.Cu) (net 7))
 (segment (start 151.6 71.3) (end 152.9 71.3) (width 0.2) (layer F.Cu) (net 7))
 (segment (start 147.15 71.1) (end 147.15 71) (width 0.2) (layer F.Cu) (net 7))
 (segment (start 152.45 70.85) (end 152.9 71.3) (width 0.15) (layer F.Cu) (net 7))
 (segment (start 148.9 71.1) (end 149.5 71.7) (width 0.2) (layer B.Cu) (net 8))
 (segment (start 149.5 71.7) (end 150.8 71.7) (width 0.2) (layer B.Cu) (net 8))
 (segment (start 150.8 71.7) (end 151.2 72.1) (width 0.2) (layer B.Cu) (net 8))
 (segment (start 151.2 72.1) (end 151.2 73.4) (width 0.2) (layer B.Cu) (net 8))
 (segment (start 151.2 73.4) (end 151.64 73.84) (width 0.2) (layer B.Cu) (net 8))
 (segment (start 151.64 73.84) (end 152.9 73.84) (width 0.2) (layer B.Cu) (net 8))
 (segment (start 149.45 71.1) (end 148.9 71.1) (width 0.2) (layer F.Cu) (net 8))
 (via (at 148.9 71.1) (size 0.6) (drill 0.3) (layers F.Cu B.Cu) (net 8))
 (segment (start 148.524999 71.674999) (end 148.05 71.2) (width 0.2) (layer F.Cu) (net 13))
 (segment (start 148.950001 71.674999) (end 148.524999 71.674999) (width 0.2) (layer F.Cu) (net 13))
 (segment (start 149.075 73.5) (end 149.075 71.799998) (width 0.2) (layer F.Cu) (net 13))
 (segment (start 149.075 71.799998) (end 148.950001 71.674999) (width 0.2) (layer F.Cu) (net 13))
 (segment (start 148.05 71.2) (end 148.05 71.1) (width 0.2) (layer F.Cu) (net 13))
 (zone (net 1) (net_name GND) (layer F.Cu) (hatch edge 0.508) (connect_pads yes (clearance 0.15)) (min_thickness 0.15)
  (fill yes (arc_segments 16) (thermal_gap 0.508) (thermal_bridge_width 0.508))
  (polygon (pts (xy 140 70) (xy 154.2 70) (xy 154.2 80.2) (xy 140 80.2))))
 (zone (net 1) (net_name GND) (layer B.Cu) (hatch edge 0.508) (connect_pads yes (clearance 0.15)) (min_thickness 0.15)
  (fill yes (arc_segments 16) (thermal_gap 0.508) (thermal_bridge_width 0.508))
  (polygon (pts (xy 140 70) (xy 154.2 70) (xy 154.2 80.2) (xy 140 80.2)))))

